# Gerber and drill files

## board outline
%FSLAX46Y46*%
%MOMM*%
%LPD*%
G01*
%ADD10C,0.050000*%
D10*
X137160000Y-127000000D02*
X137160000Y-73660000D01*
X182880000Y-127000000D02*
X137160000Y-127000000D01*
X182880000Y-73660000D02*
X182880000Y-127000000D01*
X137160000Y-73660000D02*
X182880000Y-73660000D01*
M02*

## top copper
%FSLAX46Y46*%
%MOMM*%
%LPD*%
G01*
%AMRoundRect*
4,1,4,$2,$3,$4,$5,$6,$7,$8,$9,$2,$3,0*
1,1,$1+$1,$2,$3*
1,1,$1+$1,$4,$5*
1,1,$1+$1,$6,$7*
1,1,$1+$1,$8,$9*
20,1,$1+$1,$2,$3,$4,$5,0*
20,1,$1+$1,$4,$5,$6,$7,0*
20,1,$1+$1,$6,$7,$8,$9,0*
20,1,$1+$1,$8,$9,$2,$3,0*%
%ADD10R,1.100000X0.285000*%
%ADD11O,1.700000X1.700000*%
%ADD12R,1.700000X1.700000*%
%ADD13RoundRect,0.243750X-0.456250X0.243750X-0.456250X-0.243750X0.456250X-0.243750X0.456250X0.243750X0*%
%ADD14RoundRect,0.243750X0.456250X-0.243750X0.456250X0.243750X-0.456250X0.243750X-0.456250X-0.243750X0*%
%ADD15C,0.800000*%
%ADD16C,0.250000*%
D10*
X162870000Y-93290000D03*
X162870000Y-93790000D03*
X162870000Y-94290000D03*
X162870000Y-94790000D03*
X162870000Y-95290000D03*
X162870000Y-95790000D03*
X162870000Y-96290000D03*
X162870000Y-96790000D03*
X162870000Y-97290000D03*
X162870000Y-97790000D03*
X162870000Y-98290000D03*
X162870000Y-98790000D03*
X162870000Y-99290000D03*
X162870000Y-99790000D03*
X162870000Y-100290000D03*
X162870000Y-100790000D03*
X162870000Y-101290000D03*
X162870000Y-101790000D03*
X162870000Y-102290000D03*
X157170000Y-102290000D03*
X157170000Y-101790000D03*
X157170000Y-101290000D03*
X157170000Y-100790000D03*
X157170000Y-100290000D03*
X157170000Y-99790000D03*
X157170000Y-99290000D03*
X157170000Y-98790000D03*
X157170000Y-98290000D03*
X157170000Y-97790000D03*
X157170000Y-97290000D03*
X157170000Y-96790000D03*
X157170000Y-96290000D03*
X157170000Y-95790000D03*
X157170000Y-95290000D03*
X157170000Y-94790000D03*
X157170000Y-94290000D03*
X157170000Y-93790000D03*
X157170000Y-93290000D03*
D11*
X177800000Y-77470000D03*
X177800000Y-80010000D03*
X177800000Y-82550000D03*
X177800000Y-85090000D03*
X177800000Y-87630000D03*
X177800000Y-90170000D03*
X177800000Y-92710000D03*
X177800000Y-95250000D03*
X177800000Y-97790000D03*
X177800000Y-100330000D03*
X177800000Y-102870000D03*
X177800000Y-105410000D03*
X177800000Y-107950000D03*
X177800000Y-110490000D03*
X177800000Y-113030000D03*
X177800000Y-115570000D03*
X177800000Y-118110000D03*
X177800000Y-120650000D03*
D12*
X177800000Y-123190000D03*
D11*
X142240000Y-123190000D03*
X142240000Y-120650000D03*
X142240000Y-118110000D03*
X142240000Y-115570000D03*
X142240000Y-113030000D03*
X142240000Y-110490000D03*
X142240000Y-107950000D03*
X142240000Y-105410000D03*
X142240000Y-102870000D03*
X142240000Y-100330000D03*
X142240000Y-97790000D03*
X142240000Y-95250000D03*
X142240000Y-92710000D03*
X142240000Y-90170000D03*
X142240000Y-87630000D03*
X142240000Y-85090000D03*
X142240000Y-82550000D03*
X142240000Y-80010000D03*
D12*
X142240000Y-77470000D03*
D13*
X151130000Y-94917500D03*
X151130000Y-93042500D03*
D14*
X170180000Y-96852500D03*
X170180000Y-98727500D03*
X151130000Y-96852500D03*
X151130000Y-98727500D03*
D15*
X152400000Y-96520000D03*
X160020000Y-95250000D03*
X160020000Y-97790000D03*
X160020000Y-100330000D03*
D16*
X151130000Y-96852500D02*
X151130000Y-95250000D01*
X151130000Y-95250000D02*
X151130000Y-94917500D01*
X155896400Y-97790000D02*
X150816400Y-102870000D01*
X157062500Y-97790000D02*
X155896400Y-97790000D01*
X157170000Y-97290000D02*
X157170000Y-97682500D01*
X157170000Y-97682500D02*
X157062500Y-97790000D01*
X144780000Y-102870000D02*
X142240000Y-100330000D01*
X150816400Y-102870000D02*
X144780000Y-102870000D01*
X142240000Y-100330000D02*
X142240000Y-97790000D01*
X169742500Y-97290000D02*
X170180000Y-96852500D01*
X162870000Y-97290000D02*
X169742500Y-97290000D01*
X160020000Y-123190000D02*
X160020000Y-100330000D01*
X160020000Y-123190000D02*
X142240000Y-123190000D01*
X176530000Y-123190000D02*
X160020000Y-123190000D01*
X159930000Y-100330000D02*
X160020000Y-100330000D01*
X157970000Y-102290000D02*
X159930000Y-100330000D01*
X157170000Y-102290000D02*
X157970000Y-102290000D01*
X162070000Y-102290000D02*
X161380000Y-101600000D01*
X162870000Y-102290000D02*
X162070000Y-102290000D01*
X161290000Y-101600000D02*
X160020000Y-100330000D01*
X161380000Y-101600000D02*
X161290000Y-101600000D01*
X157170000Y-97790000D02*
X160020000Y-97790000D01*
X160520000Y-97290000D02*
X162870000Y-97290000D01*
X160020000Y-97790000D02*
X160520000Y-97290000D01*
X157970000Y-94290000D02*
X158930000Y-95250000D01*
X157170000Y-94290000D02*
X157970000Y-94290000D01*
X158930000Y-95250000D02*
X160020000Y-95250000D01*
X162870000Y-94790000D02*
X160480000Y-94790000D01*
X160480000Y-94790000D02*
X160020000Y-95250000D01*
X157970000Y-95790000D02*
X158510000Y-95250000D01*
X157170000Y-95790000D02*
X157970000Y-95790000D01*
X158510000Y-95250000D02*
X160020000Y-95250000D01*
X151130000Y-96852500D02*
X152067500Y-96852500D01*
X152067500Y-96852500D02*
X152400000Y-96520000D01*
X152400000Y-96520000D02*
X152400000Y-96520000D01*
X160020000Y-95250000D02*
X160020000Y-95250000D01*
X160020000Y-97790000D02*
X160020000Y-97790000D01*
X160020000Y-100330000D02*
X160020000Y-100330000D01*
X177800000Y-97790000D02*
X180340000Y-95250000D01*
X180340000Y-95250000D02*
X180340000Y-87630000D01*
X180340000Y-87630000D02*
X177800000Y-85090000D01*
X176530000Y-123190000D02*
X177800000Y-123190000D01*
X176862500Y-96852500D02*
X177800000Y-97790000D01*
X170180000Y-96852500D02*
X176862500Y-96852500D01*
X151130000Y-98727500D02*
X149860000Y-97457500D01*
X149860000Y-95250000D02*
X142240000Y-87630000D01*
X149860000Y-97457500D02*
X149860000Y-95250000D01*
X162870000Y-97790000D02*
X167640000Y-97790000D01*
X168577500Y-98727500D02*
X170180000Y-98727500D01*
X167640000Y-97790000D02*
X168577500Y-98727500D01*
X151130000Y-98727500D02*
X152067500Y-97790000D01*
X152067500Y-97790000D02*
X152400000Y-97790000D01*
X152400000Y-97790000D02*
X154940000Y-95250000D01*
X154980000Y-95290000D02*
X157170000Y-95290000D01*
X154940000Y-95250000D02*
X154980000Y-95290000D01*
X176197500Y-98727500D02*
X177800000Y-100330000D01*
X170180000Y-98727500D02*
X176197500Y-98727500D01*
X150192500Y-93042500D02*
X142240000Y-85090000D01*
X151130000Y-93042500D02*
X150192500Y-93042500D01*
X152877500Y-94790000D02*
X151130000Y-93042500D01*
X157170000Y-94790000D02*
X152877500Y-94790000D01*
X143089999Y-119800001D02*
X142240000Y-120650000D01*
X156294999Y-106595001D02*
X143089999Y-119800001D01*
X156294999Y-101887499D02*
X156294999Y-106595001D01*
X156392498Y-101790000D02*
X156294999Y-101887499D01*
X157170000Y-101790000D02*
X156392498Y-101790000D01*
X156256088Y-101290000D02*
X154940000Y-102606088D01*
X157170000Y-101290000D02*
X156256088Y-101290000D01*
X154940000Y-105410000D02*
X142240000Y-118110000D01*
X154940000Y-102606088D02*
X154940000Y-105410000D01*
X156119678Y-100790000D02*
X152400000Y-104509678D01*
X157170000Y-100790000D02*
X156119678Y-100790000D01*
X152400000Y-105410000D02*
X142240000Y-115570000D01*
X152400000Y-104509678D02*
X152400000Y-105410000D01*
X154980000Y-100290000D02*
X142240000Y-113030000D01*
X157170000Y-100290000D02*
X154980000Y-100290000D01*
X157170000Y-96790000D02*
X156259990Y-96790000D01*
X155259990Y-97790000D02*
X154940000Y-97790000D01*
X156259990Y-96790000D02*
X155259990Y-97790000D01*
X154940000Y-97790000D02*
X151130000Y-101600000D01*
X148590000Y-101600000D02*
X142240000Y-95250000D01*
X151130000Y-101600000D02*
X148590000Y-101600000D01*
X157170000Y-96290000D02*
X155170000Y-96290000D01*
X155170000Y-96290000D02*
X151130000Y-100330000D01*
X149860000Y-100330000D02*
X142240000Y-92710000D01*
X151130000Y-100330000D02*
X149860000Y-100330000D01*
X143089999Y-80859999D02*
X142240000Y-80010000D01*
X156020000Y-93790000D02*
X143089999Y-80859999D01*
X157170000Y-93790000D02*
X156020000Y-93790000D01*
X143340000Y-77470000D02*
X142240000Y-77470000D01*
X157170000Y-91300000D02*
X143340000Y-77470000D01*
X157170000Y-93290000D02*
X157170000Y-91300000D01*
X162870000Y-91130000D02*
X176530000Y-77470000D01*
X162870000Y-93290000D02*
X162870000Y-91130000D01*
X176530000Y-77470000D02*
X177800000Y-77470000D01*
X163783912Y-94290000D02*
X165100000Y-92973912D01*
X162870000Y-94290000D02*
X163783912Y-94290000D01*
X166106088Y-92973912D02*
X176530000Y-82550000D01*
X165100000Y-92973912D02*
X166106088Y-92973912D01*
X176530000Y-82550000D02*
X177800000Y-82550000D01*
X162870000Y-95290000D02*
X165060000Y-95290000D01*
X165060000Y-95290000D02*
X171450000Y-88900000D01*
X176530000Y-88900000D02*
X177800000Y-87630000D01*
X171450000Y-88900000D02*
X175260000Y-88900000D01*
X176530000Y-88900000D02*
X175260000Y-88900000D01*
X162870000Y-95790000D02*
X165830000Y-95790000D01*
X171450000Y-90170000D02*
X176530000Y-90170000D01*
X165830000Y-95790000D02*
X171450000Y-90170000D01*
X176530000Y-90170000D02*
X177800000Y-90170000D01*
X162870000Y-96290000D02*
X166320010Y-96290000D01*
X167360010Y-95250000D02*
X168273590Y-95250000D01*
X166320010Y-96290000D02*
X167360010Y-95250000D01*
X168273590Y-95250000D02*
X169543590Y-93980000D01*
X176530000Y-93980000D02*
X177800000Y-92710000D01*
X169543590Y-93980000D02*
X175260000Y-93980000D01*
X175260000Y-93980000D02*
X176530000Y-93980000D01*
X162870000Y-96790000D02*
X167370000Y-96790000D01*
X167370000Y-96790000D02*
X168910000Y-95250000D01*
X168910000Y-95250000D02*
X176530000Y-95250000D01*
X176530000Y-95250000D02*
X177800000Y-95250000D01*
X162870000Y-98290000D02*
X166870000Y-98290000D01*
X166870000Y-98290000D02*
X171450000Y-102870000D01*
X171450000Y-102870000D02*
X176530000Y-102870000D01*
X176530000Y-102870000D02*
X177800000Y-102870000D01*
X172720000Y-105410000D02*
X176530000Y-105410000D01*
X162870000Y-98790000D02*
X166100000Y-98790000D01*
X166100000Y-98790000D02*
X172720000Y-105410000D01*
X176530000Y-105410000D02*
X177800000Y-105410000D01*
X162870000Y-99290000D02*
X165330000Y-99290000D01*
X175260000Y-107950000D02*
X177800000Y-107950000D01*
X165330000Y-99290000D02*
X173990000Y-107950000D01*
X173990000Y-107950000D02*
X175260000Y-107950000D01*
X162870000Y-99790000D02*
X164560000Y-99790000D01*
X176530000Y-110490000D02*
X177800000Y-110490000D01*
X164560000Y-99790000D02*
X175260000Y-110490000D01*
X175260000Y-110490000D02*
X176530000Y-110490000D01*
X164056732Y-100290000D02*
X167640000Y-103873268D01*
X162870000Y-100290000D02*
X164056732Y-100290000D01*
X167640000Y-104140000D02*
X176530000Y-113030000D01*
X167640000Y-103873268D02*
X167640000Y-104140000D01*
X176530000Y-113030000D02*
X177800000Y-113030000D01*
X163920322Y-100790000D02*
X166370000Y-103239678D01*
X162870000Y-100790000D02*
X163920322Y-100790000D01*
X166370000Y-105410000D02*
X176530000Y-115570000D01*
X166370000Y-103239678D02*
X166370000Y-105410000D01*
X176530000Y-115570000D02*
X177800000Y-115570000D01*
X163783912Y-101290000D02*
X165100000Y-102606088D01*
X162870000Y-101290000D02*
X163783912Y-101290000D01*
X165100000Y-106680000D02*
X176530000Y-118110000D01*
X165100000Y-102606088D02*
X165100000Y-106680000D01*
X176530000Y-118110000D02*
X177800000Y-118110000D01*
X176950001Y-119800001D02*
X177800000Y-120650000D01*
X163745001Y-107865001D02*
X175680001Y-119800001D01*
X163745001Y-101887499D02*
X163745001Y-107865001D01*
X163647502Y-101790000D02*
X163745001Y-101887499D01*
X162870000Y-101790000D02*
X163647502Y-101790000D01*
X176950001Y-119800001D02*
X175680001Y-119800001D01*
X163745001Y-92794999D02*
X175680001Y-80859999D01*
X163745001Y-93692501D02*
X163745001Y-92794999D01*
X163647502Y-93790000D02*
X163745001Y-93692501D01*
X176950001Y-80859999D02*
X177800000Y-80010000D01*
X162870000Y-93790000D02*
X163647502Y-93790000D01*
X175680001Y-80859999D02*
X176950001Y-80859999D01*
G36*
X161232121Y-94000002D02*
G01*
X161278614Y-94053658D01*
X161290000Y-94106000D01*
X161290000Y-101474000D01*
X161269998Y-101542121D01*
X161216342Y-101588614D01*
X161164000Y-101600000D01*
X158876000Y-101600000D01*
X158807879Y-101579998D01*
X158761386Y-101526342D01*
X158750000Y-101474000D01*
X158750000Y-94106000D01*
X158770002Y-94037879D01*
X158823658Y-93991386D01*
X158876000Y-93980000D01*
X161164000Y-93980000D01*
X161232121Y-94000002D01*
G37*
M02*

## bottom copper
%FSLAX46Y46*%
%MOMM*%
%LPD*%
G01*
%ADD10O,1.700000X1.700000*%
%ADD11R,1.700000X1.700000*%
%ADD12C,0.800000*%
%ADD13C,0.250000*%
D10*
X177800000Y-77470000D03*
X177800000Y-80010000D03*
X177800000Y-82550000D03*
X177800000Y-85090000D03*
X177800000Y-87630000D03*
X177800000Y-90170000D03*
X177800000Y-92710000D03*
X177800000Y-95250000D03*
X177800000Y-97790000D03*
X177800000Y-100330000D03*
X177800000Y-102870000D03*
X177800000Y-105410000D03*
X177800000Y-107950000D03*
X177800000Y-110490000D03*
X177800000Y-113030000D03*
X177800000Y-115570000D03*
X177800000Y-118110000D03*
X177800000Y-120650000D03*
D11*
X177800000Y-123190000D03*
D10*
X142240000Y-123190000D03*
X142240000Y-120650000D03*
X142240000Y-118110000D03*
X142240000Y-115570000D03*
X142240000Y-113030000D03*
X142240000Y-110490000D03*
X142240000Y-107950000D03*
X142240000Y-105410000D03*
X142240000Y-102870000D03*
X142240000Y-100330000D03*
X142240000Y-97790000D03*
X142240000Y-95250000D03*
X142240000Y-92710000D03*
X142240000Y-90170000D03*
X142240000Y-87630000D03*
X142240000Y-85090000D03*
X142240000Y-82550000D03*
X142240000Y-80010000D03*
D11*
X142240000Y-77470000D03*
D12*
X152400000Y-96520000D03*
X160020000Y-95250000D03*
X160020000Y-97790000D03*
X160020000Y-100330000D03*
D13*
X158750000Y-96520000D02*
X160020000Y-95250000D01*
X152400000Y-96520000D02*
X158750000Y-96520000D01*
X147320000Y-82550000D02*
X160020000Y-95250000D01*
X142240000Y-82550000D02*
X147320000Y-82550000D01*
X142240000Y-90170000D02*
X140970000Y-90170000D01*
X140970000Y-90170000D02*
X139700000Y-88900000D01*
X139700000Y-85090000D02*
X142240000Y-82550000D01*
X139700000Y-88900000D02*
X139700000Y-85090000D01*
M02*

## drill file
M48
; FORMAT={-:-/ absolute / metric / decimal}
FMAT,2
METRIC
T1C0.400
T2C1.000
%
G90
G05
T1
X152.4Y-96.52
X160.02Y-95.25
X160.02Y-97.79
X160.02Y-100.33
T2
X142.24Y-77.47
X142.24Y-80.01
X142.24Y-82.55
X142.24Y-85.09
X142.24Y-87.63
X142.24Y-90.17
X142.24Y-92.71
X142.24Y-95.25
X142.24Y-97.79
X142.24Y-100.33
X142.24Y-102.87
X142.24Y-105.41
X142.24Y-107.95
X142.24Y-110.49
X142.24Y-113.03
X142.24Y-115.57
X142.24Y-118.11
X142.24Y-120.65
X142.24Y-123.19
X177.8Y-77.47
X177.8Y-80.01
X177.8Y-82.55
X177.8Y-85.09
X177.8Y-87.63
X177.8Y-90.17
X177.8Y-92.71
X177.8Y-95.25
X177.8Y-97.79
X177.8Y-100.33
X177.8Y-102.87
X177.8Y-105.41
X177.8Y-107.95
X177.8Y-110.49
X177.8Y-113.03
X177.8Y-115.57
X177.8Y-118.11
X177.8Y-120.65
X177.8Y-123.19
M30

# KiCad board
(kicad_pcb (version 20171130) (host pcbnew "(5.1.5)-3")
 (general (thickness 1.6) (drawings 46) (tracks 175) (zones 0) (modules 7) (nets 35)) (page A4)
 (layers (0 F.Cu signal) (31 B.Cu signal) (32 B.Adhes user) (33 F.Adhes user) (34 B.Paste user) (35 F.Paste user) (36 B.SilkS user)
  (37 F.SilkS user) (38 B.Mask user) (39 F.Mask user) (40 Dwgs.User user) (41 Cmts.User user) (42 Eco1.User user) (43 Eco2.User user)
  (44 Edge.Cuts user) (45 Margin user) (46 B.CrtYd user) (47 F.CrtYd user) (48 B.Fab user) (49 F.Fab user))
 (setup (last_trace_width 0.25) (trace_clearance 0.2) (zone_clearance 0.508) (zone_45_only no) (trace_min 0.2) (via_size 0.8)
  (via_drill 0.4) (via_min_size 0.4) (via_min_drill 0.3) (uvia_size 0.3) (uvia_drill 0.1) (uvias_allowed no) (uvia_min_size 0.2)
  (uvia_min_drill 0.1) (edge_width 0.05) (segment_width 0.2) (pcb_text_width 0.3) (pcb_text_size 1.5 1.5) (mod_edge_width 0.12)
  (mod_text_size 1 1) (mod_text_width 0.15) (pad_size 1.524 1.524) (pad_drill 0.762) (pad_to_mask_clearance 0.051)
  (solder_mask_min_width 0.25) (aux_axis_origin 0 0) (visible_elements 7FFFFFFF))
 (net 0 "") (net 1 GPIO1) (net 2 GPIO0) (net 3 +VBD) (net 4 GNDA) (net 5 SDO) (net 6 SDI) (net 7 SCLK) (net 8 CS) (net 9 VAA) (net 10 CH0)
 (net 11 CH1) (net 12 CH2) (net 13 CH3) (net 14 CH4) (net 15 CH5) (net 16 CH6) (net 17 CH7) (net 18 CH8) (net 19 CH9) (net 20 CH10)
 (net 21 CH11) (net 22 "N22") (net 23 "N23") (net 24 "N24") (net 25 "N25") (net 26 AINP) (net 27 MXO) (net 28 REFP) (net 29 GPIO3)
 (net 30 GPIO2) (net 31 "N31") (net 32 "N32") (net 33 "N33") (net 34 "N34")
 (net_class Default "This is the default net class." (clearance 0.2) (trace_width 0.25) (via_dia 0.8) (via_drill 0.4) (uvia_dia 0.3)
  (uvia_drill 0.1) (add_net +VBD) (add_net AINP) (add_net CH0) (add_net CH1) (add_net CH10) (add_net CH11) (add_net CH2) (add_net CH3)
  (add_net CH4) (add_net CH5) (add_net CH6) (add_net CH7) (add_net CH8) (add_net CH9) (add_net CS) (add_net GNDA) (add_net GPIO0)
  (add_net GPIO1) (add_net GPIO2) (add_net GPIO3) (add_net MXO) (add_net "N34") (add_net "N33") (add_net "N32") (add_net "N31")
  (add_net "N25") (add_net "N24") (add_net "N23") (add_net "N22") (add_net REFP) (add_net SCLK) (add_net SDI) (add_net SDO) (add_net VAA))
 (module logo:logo (layer F.Cu) (at 160.02 82.55)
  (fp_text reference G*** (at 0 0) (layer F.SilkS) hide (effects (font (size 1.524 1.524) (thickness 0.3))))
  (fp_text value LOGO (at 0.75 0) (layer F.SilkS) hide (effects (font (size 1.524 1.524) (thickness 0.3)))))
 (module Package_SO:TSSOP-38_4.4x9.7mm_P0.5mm (layer F.Cu) (at 160.02 97.79)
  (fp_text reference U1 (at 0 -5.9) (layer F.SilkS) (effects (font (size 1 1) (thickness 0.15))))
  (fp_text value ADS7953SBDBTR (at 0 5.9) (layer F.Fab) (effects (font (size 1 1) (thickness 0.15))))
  (pad 38 smd rect (at 2.85 -4.5) (size 1.1 0.285) (layers F.Cu F.Paste F.Mask) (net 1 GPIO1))
  (pad 37 smd rect (at 2.85 -4) (size 1.1 0.285) (layers F.Cu F.Paste F.Mask) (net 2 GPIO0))
  (pad 36 smd rect (at 2.85 -3.5) (size 1.1 0.285) (layers F.Cu F.Paste F.Mask) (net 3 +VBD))
  (pad 35 smd rect (at 2.85 -3) (size 1.1 0.285) (layers F.Cu F.Paste F.Mask) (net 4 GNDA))
  (pad 34 smd rect (at 2.85 -2.5) (size 1.1 0.285) (layers F.Cu F.Paste F.Mask) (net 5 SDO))
  (pad 33 smd rect (at 2.85 -2) (size 1.1 0.285) (layers F.Cu F.Paste F.Mask) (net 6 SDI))
  (pad 32 smd rect (at 2.85 -1.5) (size 1.1 0.285) (layers F.Cu F.Paste F.Mask) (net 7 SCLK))
  (pad 31 smd rect (at 2.85 -1) (size 1.1 0.285) (layers F.Cu F.Paste F.Mask) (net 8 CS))
  (pad 30 smd rect (at 2.85 -0.5) (size 1.1 0.285) (layers F.Cu F.Paste F.Mask) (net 4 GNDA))
  (pad 29 smd rect (at 2.85 0) (size 1.1 0.285) (layers F.Cu F.Paste F.Mask) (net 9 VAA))
  (pad 28 smd rect (at 2.85 0.5) (size 1.1 0.285) (layers F.Cu F.Paste F.Mask) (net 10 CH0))
  (pad 27 smd rect (at 2.85 1) (size 1.1 0.285) (layers F.Cu F.Paste F.Mask) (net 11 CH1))
  (pad 26 smd rect (at 2.85 1.5) (size 1.1 0.285) (layers F.Cu F.Paste F.Mask) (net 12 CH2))
  (pad 25 smd rect (at 2.85 2) (size 1.1 0.285) (layers F.Cu F.Paste F.Mask) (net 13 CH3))
  (pad 24 smd rect (at 2.85 2.5) (size 1.1 0.285) (layers F.Cu F.Paste F.Mask) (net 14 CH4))
  (pad 23 smd rect (at 2.85 3) (size 1.1 0.285) (layers F.Cu F.Paste F.Mask) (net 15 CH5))
  (pad 22 smd rect (at 2.85 3.5) (size 1.1 0.285) (layers F.Cu F.Paste F.Mask) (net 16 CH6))
  (pad 21 smd rect (at 2.85 4) (size 1.1 0.285) (layers F.Cu F.Paste F.Mask) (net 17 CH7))
  (pad 20 smd rect (at 2.85 4.5) (size 1.1 0.285) (layers F.Cu F.Paste F.Mask) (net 4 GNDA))
  (pad 19 smd rect (at -2.85 4.5) (size 1.1 0.285) (layers F.Cu F.Paste F.Mask) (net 4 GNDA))
  (pad 18 smd rect (at -2.85 4) (size 1.1 0.285) (layers F.Cu F.Paste F.Mask) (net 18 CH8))
  (pad 17 smd rect (at -2.85 3.5) (size 1.1 0.285) (layers F.Cu F.Paste F.Mask) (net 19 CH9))
  (pad 16 smd rect (at -2.85 3) (size 1.1 0.285) (layers F.Cu F.Paste F.Mask) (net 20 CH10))
  (pad 15 smd rect (at -2.85 2.5) (size 1.1 0.285) (layers F.Cu F.Paste F.Mask) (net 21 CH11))
  (pad 14 smd rect (at -2.85 2) (size 1.1 0.285) (layers F.Cu F.Paste F.Mask) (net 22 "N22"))
  (pad 13 smd rect (at -2.85 1.5) (size 1.1 0.285) (layers F.Cu F.Paste F.Mask) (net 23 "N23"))
  (pad 12 smd rect (at -2.85 1) (size 1.1 0.285) (layers F.Cu F.Paste F.Mask) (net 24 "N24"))
  (pad 11 smd rect (at -2.85 0.5) (size 1.1 0.285) (layers F.Cu F.Paste F.Mask) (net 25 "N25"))
  (pad 10 smd rect (at -2.85 0) (size 1.1 0.285) (layers F.Cu F.Paste F.Mask) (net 4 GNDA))
  (pad 9 smd rect (at -2.85 -0.5) (size 1.1 0.285) (layers F.Cu F.Paste F.Mask) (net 4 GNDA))
  (pad 8 smd rect (at -2.85 -1) (size 1.1 0.285) (layers F.Cu F.Paste F.Mask) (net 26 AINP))
  (pad 7 smd rect (at -2.85 -1.5) (size 1.1 0.285) (layers F.Cu F.Paste F.Mask) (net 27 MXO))
  (pad 6 smd rect (at -2.85 -2) (size 1.1 0.285) (layers F.Cu F.Paste F.Mask) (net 4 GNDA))
  (pad 5 smd rect (at -2.85 -2.5) (size 1.1 0.285) (layers F.Cu F.Paste F.Mask) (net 9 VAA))
  (pad 4 smd rect (at -2.85 -3) (size 1.1 0.285) (layers F.Cu F.Paste F.Mask) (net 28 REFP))
  (pad 3 smd rect (at -2.85 -3.5) (size 1.1 0.285) (layers F.Cu F.Paste F.Mask) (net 4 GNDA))
  (pad 2 smd rect (at -2.85 -4) (size 1.1 0.285) (layers F.Cu F.Paste F.Mask) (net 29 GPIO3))
  (pad 1 smd rect (at -2.85 -4.5) (size 1.1 0.285) (layers F.Cu F.Paste F.Mask) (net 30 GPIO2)))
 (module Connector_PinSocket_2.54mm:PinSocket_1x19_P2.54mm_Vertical (layer F.Cu) (at 177.8 123.19 180)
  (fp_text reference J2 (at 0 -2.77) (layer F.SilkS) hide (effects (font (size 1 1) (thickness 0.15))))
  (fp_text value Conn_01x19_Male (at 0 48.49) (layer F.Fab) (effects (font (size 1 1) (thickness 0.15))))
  (pad 19 thru_hole oval (at 0 45.72 180) (size 1.7 1.7) (drill 1) (layers *.Cu *.Mask) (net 1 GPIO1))
  (pad 18 thru_hole oval (at 0 43.18 180) (size 1.7 1.7) (drill 1) (layers *.Cu *.Mask) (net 2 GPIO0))
  (pad 17 thru_hole oval (at 0 40.64 180) (size 1.7 1.7) (drill 1) (layers *.Cu *.Mask) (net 3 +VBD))
  (pad 16 thru_hole oval (at 0 38.1 180) (size 1.7 1.7) (drill 1) (layers *.Cu *.Mask) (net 4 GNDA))
  (pad 15 thru_hole oval (at 0 35.56 180) (size 1.7 1.7) (drill 1) (layers *.Cu *.Mask) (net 5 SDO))
  (pad 14 thru_hole oval (at 0 33.02 180) (size 1.7 1.7) (drill 1) (layers *.Cu *.Mask) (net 6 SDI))
  (pad 13 thru_hole oval (at 0 30.48 180) (size 1.7 1.7) (drill 1) (layers *.Cu *.Mask) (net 7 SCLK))
  (pad 12 thru_hole oval (at 0 27.94 180) (size 1.7 1.7) (drill 1) (layers *.Cu *.Mask) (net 8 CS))
  (pad 11 thru_hole oval (at 0 25.4 180) (size 1.7 1.7) (drill 1) (layers *.Cu *.Mask) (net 4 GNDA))
  (pad 10 thru_hole oval (at 0 22.86 180) (size 1.7 1.7) (drill 1) (layers *.Cu *.Mask) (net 9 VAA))
  (pad 9 thru_hole oval (at 0 20.32 180) (size 1.7 1.7) (drill 1) (layers *.Cu *.Mask) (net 10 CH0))
  (pad 8 thru_hole oval (at 0 17.78 180) (size 1.7 1.7) (drill 1) (layers *.Cu *.Mask) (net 11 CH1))
  (pad 7 thru_hole oval (at 0 15.24 180) (size 1.7 1.7) (drill 1) (layers *.Cu *.Mask) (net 12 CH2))
  (pad 6 thru_hole oval (at 0 12.7 180) (size 1.7 1.7) (drill 1) (layers *.Cu *.Mask) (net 13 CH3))
  (pad 5 thru_hole oval (at 0 10.16 180) (size 1.7 1.7) (drill 1) (layers *.Cu *.Mask) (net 14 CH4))
  (pad 4 thru_hole oval (at 0 7.62 180) (size 1.7 1.7) (drill 1) (layers *.Cu *.Mask) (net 15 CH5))
  (pad 3 thru_hole oval (at 0 5.08 180) (size 1.7 1.7) (drill 1) (layers *.Cu *.Mask) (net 16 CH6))
  (pad 2 thru_hole oval (at 0 2.54 180) (size 1.7 1.7) (drill 1) (layers *.Cu *.Mask) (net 17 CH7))
  (pad 1 thru_hole rect (at 0 0 180) (size 1.7 1.7) (drill 1) (layers *.Cu *.Mask) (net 4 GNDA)))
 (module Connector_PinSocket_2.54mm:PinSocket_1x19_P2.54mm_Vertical (layer F.Cu) (at 142.24 77.47)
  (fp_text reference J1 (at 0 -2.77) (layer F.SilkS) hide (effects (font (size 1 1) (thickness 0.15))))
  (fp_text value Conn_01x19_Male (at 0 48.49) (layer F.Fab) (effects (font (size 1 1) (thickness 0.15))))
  (pad 19 thru_hole oval (at 0 45.72) (size 1.7 1.7) (drill 1) (layers *.Cu *.Mask) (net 4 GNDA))
  (pad 18 thru_hole oval (at 0 43.18) (size 1.7 1.7) (drill 1) (layers *.Cu *.Mask) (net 18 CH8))
  (pad 17 thru_hole oval (at 0 40.64) (size 1.7 1.7) (drill 1) (layers *.Cu *.Mask) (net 19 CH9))
  (pad 16 thru_hole oval (at 0 38.1) (size 1.7 1.7) (drill 1) (layers *.Cu *.Mask) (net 20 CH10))
  (pad 15 thru_hole oval (at 0 35.56) (size 1.7 1.7) (drill 1) (layers *.Cu *.Mask) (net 21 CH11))
  (pad 14 thru_hole oval (at 0 33.02) (size 1.7 1.7) (drill 1) (layers *.Cu *.Mask) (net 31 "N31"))
  (pad 13 thru_hole oval (at 0 30.48) (size 1.7 1.7) (drill 1) (layers *.Cu *.Mask) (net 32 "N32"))
  (pad 12 thru_hole oval (at 0 27.94) (size 1.7 1.7) (drill 1) (layers *.Cu *.Mask) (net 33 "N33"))
  (pad 11 thru_hole oval (at 0 25.4) (size 1.7 1.7) (drill 1) (layers *.Cu *.Mask) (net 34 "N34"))
  (pad 10 thru_hole oval (at 0 22.86) (size 1.7 1.7) (drill 1) (layers *.Cu *.Mask) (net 4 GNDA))
  (pad 9 thru_hole oval (at 0 20.32) (size 1.7 1.7) (drill 1) (layers *.Cu *.Mask) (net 4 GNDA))
  (pad 8 thru_hole oval (at 0 17.78) (size 1.7 1.7) (drill 1) (layers *.Cu *.Mask) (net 26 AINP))
  (pad 7 thru_hole oval (at 0 15.24) (size 1.7 1.7) (drill 1) (layers *.Cu *.Mask) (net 27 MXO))
  (pad 6 thru_hole oval (at 0 12.7) (size 1.7 1.7) (drill 1) (layers *.Cu *.Mask) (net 4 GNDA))
  (pad 5 thru_hole oval (at 0 10.16) (size 1.7 1.7) (drill 1) (layers *.Cu *.Mask) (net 9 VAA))
  (pad 4 thru_hole oval (at 0 7.62) (size 1.7 1.7) (drill 1) (layers *.Cu *.Mask) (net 28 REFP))
  (pad 3 thru_hole oval (at 0 5.08) (size 1.7 1.7) (drill 1) (layers *.Cu *.Mask) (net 4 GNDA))
  (pad 2 thru_hole oval (at 0 2.54) (size 1.7 1.7) (drill 1) (layers *.Cu *.Mask) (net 29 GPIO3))
  (pad 1 thru_hole rect (at 0 0) (size 1.7 1.7) (drill 1) (layers *.Cu *.Mask) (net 30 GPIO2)))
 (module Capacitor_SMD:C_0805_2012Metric (layer F.Cu) (at 151.13 93.98 270)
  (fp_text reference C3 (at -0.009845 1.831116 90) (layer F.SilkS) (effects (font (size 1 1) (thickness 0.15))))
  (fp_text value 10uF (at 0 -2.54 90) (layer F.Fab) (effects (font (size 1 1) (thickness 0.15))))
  (pad 2 smd roundrect (at 0.9375 0 270) (size 0.975 1.4) (layers F.Cu F.Paste F.Mask) (roundrect_rratio 0.25) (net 4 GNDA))
  (pad 1 smd roundrect (at -0.9375 0 270) (size 0.975 1.4) (layers F.Cu F.Paste F.Mask) (roundrect_rratio 0.25) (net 28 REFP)))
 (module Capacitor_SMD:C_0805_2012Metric (layer F.Cu) (at 170.18 97.79 90)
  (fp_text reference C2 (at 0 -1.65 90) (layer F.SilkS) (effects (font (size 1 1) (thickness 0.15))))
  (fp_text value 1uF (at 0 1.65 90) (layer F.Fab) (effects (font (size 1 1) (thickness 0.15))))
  (pad 2 smd roundrect (at 0.9375 0 90) (size 0.975 1.4) (layers F.Cu F.Paste F.Mask) (roundrect_rratio 0.25) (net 4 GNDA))
  (pad 1 smd roundrect (at -0.9375 0 90) (size 0.975 1.4) (layers F.Cu F.Paste F.Mask) (roundrect_rratio 0.25) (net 9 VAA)))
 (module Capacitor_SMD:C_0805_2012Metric (layer F.Cu) (at 151.13 97.79 90)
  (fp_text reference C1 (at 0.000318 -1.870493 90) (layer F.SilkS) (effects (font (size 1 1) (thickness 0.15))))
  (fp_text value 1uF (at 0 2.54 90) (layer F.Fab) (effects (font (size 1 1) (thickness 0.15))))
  (pad 2 smd roundrect (at 0.9375 0 90) (size 0.975 1.4) (layers F.Cu F.Paste F.Mask) (roundrect_rratio 0.25) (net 4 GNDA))
  (pad 1 smd roundrect (at -0.9375 0 90) (size 0.975 1.4) (layers F.Cu F.Paste F.Mask) (roundrect_rratio 0.25) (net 9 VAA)))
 (gr_line (start 137.16 127) (end 137.16 73.66) (layer Edge.Cuts) (width 0.05))
 (gr_line (start 182.88 127) (end 137.16 127) (layer Edge.Cuts) (width 0.05))
 (gr_line (start 182.88 73.66) (end 182.88 127) (layer Edge.Cuts) (width 0.05))
 (gr_line (start 137.16 73.66) (end 182.88 73.66) (layer Edge.Cuts) (width 0.05))
 (segment (start 151.13 96.8525) (end 151.13 95.25) (width 0.25) (layer F.Cu) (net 4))
 (segment (start 151.13 95.25) (end 151.13 94.9175) (width 0.25) (layer F.Cu) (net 4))
 (segment (start 155.8964 97.79) (end 150.8164 102.87) (width 0.25) (layer F.Cu) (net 4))
 (segment (start 157.0625 97.79) (end 155.8964 97.79) (width 0.25) (layer F.Cu) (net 4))
 (segment (start 157.17 97.29) (end 157.17 97.6825) (width 0.25) (layer F.Cu) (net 4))
 (segment (start 157.17 97.6825) (end 157.0625 97.79) (width 0.25) (layer F.Cu) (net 4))
 (segment (start 144.78 102.87) (end 142.24 100.33) (width 0.25) (layer F.Cu) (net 4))
 (segment (start 150.8164 102.87) (end 144.78 102.87) (width 0.25) (layer F.Cu) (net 4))
 (segment (start 142.24 100.33) (end 142.24 97.79) (width 0.25) (layer F.Cu) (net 4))
 (segment (start 169.7425 97.29) (end 170.18 96.8525) (width 0.25) (layer F.Cu) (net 4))
 (segment (start 162.87 97.29) (end 169.7425 97.29) (width 0.25) (layer F.Cu) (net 4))
 (segment (start 160.02 123.19) (end 160.02 100.33) (width 0.25) (layer F.Cu) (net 4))
 (segment (start 160.02 123.19) (end 142.24 123.19) (width 0.25) (layer F.Cu) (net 4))
 (segment (start 176.53 123.19) (end 160.02 123.19) (width 0.25) (layer F.Cu) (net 4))
 (segment (start 159.93 100.33) (end 160.02 100.33) (width 0.25) (layer F.Cu) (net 4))
 (segment (start 157.97 102.29) (end 159.93 100.33) (width 0.25) (layer F.Cu) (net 4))
 (segment (start 157.17 102.29) (end 157.97 102.29) (width 0.25) (layer F.Cu) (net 4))
 (segment (start 162.07 102.29) (end 161.38 101.6) (width 0.25) (layer F.Cu) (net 4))
 (segment (start 162.87 102.29) (end 162.07 102.29) (width 0.25) (layer F.Cu) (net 4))
 (segment (start 161.29 101.6) (end 160.02 100.33) (width 0.25) (layer F.Cu) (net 4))
 (segment (start 161.38 101.6) (end 161.29 101.6) (width 0.25) (layer F.Cu) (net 4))
 (segment (start 157.17 97.79) (end 160.02 97.79) (width 0.25) (layer F.Cu) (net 4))
 (segment (start 160.52 97.29) (end 162.87 97.29) (width 0.25) (layer F.Cu) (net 4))
 (segment (start 160.02 97.79) (end 160.52 97.29) (width 0.25) (layer F.Cu) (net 4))
 (segment (start 157.97 94.29) (end 158.93 95.25) (width 0.25) (layer F.Cu) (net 4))
 (segment (start 157.17 94.29) (end 157.97 94.29) (width 0.25) (layer F.Cu) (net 4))
 (segment (start 158.93 95.25) (end 160.02 95.25) (width 0.25) (layer F.Cu) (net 4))
 (segment (start 162.87 94.79) (end 160.48 94.79) (width 0.25) (layer F.Cu) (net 4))
 (segment (start 160.48 94.79) (end 160.02 95.25) (width 0.25) (layer F.Cu) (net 4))
 (segment (start 157.97 95.79) (end 158.51 95.25) (width 0.25) (layer F.Cu) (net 4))
 (segment (start 157.17 95.79) (end 157.97 95.79) (width 0.25) (layer F.Cu) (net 4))
 (segment (start 158.51 95.25) (end 160.02 95.25) (width 0.25) (layer F.Cu) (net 4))
 (segment (start 151.13 96.8525) (end 152.0675 96.8525) (width 0.25) (layer F.Cu) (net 4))
 (segment (start 152.0675 96.8525) (end 152.4 96.52) (width 0.25) (layer F.Cu) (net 4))
 (segment (start 152.4 96.52) (end 152.4 96.52) (width 0.25) (layer F.Cu) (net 4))
 (via (at 152.4 96.52) (size 0.8) (drill 0.4) (layers F.Cu B.Cu) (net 4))
 (segment (start 160.02 95.25) (end 160.02 95.25) (width 0.25) (layer F.Cu) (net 4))
 (via (at 160.02 95.25) (size 0.8) (drill 0.4) (layers F.Cu B.Cu) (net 4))
 (segment (start 160.02 97.79) (end 160.02 97.79) (width 0.25) (layer F.Cu) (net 4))
 (via (at 160.02 97.79) (size 0.8) (drill 0.4) (layers F.Cu B.Cu) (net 4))
 (segment (start 160.02 100.33) (end 160.02 100.33) (width 0.25) (layer F.Cu) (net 4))
 (via (at 160.02 100.33) (size 0.8) (drill 0.4) (layers F.Cu B.Cu) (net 4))
 (segment (start 158.75 96.52) (end 160.02 95.25) (width 0.25) (layer B.Cu) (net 4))
 (segment (start 152.4 96.52) (end 158.75 96.52) (width 0.25) (layer B.Cu) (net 4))
 (segment (start 147.32 82.55) (end 160.02 95.25) (width 0.25) (layer B.Cu) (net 4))
 (segment (start 142.24 82.55) (end 147.32 82.55) (width 0.25) (layer B.Cu) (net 4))
 (segment (start 142.24 90.17) (end 140.97 90.17) (width 0.25) (layer B.Cu) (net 4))
 (segment (start 140.97 90.17) (end 139.7 88.9) (width 0.25) (layer B.Cu) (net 4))
 (segment (start 139.7 85.09) (end 142.24 82.55) (width 0.25) (layer B.Cu) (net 4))
 (segment (start 139.7 88.9) (end 139.7 85.09) (width 0.25) (layer B.Cu) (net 4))
 (segment (start 177.8 97.79) (end 180.34 95.25) (width 0.25) (layer F.Cu) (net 4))
 (segment (start 180.34 95.25) (end 180.34 87.63) (width 0.25) (layer F.Cu) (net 4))
 (segment (start 180.34 87.63) (end 177.8 85.09) (width 0.25) (layer F.Cu) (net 4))
 (segment (start 176.53 123.19) (end 177.8 123.19) (width 0.25) (layer F.Cu) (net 4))
 (segment (start 176.8625 96.8525) (end 177.8 97.79) (width 0.25) (layer F.Cu) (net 4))
 (segment (start 170.18 96.8525) (end 176.8625 96.8525) (width 0.25) (layer F.Cu) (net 4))
 (segment (start 151.13 98.7275) (end 149.86 97.4575) (width 0.25) (layer F.Cu) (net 9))
 (segment (start 149.86 95.25) (end 142.24 87.63) (width 0.25) (layer F.Cu) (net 9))
 (segment (start 149.86 97.4575) (end 149.86 95.25) (width 0.25) (layer F.Cu) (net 9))
 (segment (start 162.87 97.79) (end 167.64 97.79) (width 0.25) (layer F.Cu) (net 9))
 (segment (start 168.5775 98.7275) (end 170.18 98.7275) (width 0.25) (layer F.Cu) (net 9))
 (segment (start 167.64 97.79) (end 168.5775 98.7275) (width 0.25) (layer F.Cu) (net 9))
 (segment (start 151.13 98.7275) (end 152.0675 97.79) (width 0.25) (layer F.Cu) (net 9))
 (segment (start 152.0675 97.79) (end 152.4 97.79) (width 0.25) (layer F.Cu) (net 9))
 (segment (start 152.4 97.79) (end 154.94 95.25) (width 0.25) (layer F.Cu) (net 9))
 (segment (start 154.98 95.29) (end 157.17 95.29) (width 0.25) (layer F.Cu) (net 9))
 (segment (start 154.94 95.25) (end 154.98 95.29) (width 0.25) (layer F.Cu) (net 9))
 (segment (start 176.1975 98.7275) (end 177.8 100.33) (width 0.25) (layer F.Cu) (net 9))
 (segment (start 170.18 98.7275) (end 176.1975 98.7275) (width 0.25) (layer F.Cu) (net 9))
 (segment (start 150.1925 93.0425) (end 142.24 85.09) (width 0.25) (layer F.Cu) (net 28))
 (segment (start 151.13 93.0425) (end 150.1925 93.0425) (width 0.25) (layer F.Cu) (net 28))
 (segment (start 152.8775 94.79) (end 151.13 93.0425) (width 0.25) (layer F.Cu) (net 28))
 (segment (start 157.17 94.79) (end 152.8775 94.79) (width 0.25) (layer F.Cu) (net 28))
 (segment (start 143.089999 119.800001) (end 142.24 120.65) (width 0.25) (layer F.Cu) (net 18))
 (segment (start 156.294999 106.595001) (end 143.089999 119.800001) (width 0.25) (layer F.Cu) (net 18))
 (segment (start 156.294999 101.887499) (end 156.294999 106.595001) (width 0.25) (layer F.Cu) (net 18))
 (segment (start 156.392498 101.79) (end 156.294999 101.887499) (width 0.25) (layer F.Cu) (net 18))
 (segment (start 157.17 101.79) (end 156.392498 101.79) (width 0.25) (layer F.Cu) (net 18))
 (segment (start 156.256088 101.29) (end 154.94 102.606088) (width 0.25) (layer F.Cu) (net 19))
 (segment (start 157.17 101.29) (end 156.256088 101.29) (width 0.25) (layer F.Cu) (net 19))
 (segment (start 154.94 105.41) (end 142.24 118.11) (width 0.25) (layer F.Cu) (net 19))
 (segment (start 154.94 102.606088) (end 154.94 105.41) (width 0.25) (layer F.Cu) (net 19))
 (segment (start 156.119678 100.79) (end 152.4 104.509678) (width 0.25) (layer F.Cu) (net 20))
 (segment (start 157.17 100.79) (end 156.119678 100.79) (width 0.25) (layer F.Cu) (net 20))
 (segment (start 152.4 105.41) (end 142.24 115.57) (width 0.25) (layer F.Cu) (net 20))
 (segment (start 152.4 104.509678) (end 152.4 105.41) (width 0.25) (layer F.Cu) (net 20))
 (segment (start 154.98 100.29) (end 142.24 113.03) (width 0.25) (layer F.Cu) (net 21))
 (segment (start 157.17 100.29) (end 154.98 100.29) (width 0.25) (layer F.Cu) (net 21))
 (segment (start 157.17 96.79) (end 156.25999 96.79) (width 0.25) (layer F.Cu) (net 26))
 (segment (start 155.25999 97.79) (end 154.94 97.79) (width 0.25) (layer F.Cu) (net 26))
 (segment (start 156.25999 96.79) (end 155.25999 97.79) (width 0.25) (layer F.Cu) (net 26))
 (segment (start 154.94 97.79) (end 151.13 101.6) (width 0.25) (layer F.Cu) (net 26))
 (segment (start 148.59 101.6) (end 142.24 95.25) (width 0.25) (layer F.Cu) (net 26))
 (segment (start 151.13 101.6) (end 148.59 101.6) (width 0.25) (layer F.Cu) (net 26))
 (segment (start 157.17 96.29) (end 155.17 96.29) (width 0.25) (layer F.Cu) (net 27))
 (segment (start 155.17 96.29) (end 151.13 100.33) (width 0.25) (layer F.Cu) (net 27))
 (segment (start 149.86 100.33) (end 142.24 92.71) (width 0.25) (layer F.Cu) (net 27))
 (segment (start 151.13 100.33) (end 149.86 100.33) (width 0.25) (layer F.Cu) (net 27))
 (segment (start 143.089999 80.859999) (end 142.24 80.01) (width 0.25) (layer F.Cu) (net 29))
 (segment (start 156.02 93.79) (end 143.089999 80.859999) (width 0.25) (layer F.Cu) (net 29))
 (segment (start 157.17 93.79) (end 156.02 93.79) (width 0.25) (layer F.Cu) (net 29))
 (segment (start 143.34 77.47) (end 142.24 77.47) (width 0.25) (layer F.Cu) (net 30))
 (segment (start 157.17 91.3) (end 143.34 77.47) (width 0.25) (layer F.Cu) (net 30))
 (segment (start 157.17 93.29) (end 157.17 91.3) (width 0.25) (layer F.Cu) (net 30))
 (segment (start 162.87 91.13) (end 176.53 77.47) (width 0.25) (layer F.Cu) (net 1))
 (segment (start 162.87 93.29) (end 162.87 91.13) (width 0.25) (layer F.Cu) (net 1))
 (segment (start 176.53 77.47) (end 177.8 77.47) (width 0.25) (layer F.Cu) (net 1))
 (segment (start 163.783912 94.29) (end 165.1 92.973912) (width 0.25) (layer F.Cu) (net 3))
 (segment (start 162.87 94.29) (end 163.783912 94.29) (width 0.25) (layer F.Cu) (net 3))
 (segment (start 166.106088 92.973912) (end 176.53 82.55) (width 0.25) (layer F.Cu) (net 3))
 (segment (start 165.1 92.973912) (end 166.106088 92.973912) (width 0.25) (layer F.Cu) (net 3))
 (segment (start 176.53 82.55) (end 177.8 82.55) (width 0.25) (layer F.Cu) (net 3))
 (segment (start 162.87 95.29) (end 165.06 95.29) (width 0.25) (layer F.Cu) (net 5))
 (segment (start 165.06 95.29) (end 171.45 88.9) (width 0.25) (layer F.Cu) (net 5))
 (segment (start 176.53 88.9) (end 177.8 87.63) (width 0.25) (layer F.Cu) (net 5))
 (segment (start 171.45 88.9) (end 175.26 88.9) (width 0.25) (layer F.Cu) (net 5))
 (segment (start 176.53 88.9) (end 175.26 88.9) (width 0.25) (layer F.Cu) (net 5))
 (segment (start 162.87 95.79) (end 165.83 95.79) (width 0.25) (layer F.Cu) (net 6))
 (segment (start 171.45 90.17) (end 176.53 90.17) (width 0.25) (layer F.Cu) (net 6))
 (segment (start 165.83 95.79) (end 171.45 90.17) (width 0.25) (layer F.Cu) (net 6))
 (segment (start 176.53 90.17) (end 177.8 90.17) (width 0.25) (layer F.Cu) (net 6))
 (segment (start 162.87 96.29) (end 166.32001 96.29) (width 0.25) (layer F.Cu) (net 7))
 (segment (start 167.36001 95.25) (end 168.27359 95.25) (width 0.25) (layer F.Cu) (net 7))
 (segment (start 166.32001 96.29) (end 167.36001 95.25) (width 0.25) (layer F.Cu) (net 7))
 (segment (start 168.27359 95.25) (end 169.54359 93.98) (width 0.25) (layer F.Cu) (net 7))
 (segment (start 176.53 93.98) (end 177.8 92.71) (width 0.25) (layer F.Cu) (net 7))
 (segment (start 169.54359 93.98) (end 175.26 93.98) (width 0.25) (layer F.Cu) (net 7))
 (segment (start 175.26 93.98) (end 176.53 93.98) (width 0.25) (layer F.Cu) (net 7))
 (segment (start 162.87 96.79) (end 167.37 96.79) (width 0.25) (layer F.Cu) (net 8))
 (segment (start 167.37 96.79) (end 168.91 95.25) (width 0.25) (layer F.Cu) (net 8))
 (segment (start 168.91 95.25) (end 176.53 95.25) (width 0.25) (layer F.Cu) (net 8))
 (segment (start 176.53 95.25) (end 177.8 95.25) (width 0.25) (layer F.Cu) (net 8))
 (segment (start 162.87 98.29) (end 166.87 98.29) (width 0.25) (layer F.Cu) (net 10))
 (segment (start 166.87 98.29) (end 171.45 102.87) (width 0.25) (layer F.Cu) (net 10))
 (segment (start 171.45 102.87) (end 176.53 102.87) (width 0.25) (layer F.Cu) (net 10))
 (segment (start 176.53 102.87) (end 177.8 102.87) (width 0.25) (layer F.Cu) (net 10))
 (segment (start 172.72 105.41) (end 176.53 105.41) (width 0.25) (layer F.Cu) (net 11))
 (segment (start 162.87 98.79) (end 166.1 98.79) (width 0.25) (layer F.Cu) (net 11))
 (segment (start 166.1 98.79) (end 172.72 105.41) (width 0.25) (layer F.Cu) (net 11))
 (segment (start 176.53 105.41) (end 177.8 105.41) (width 0.25) (layer F.Cu) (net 11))
 (segment (start 162.87 99.29) (end 165.33 99.29) (width 0.25) (layer F.Cu) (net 12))
 (segment (start 175.26 107.95) (end 177.8 107.95) (width 0.25) (layer F.Cu) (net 12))
 (segment (start 165.33 99.29) (end 173.99 107.95) (width 0.25) (layer F.Cu) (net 12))
 (segment (start 173.99 107.95) (end 175.26 107.95) (width 0.25) (layer F.Cu) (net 12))
 (segment (start 162.87 99.79) (end 164.56 99.79) (width 0.25) (layer F.Cu) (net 13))
 (segment (start 176.53 110.49) (end 177.8 110.49) (width 0.25) (layer F.Cu) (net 13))
 (segment (start 164.56 99.79) (end 175.26 110.49) (width 0.25) (layer F.Cu) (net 13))
 (segment (start 175.26 110.49) (end 176.53 110.49) (width 0.25) (layer F.Cu) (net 13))
 (segment (start 164.056732 100.29) (end 167.64 103.873268) (width 0.25) (layer F.Cu) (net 14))
 (segment (start 162.87 100.29) (end 164.056732 100.29) (width 0.25) (layer F.Cu) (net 14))
 (segment (start 167.64 104.14) (end 176.53 113.03) (width 0.25) (layer F.Cu) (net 14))
 (segment (start 167.64 103.873268) (end 167.64 104.14) (width 0.25) (layer F.Cu) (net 14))
 (segment (start 176.53 113.03) (end 177.8 113.03) (width 0.25) (layer F.Cu) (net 14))
 (segment (start 163.920322 100.79) (end 166.37 103.239678) (width 0.25) (layer F.Cu) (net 15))
 (segment (start 162.87 100.79) (end 163.920322 100.79) (width 0.25) (layer F.Cu) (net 15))
 (segment (start 166.37 105.41) (end 176.53 115.57) (width 0.25) (layer F.Cu) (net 15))
 (segment (start 166.37 103.239678) (end 166.37 105.41) (width 0.25) (layer F.Cu) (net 15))
 (segment (start 176.53 115.57) (end 177.8 115.57) (width 0.25) (layer F.Cu) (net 15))
 (segment (start 163.783912 101.29) (end 165.1 102.606088) (width 0.25) (layer F.Cu) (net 16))
 (segment (start 162.87 101.29) (end 163.783912 101.29) (width 0.25) (layer F.Cu) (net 16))
 (segment (start 165.1 106.68) (end 176.53 118.11) (width 0.25) (layer F.Cu) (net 16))
 (segment (start 165.1 102.606088) (end 165.1 106.68) (width 0.25) (layer F.Cu) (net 16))
 (segment (start 176.53 118.11) (end 177.8 118.11) (width 0.25) (layer F.Cu) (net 16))
 (segment (start 176.950001 119.800001) (end 177.8 120.65) (width 0.25) (layer F.Cu) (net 17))
 (segment (start 163.745001 107.865001) (end 175.680001 119.800001) (width 0.25) (layer F.Cu) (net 17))
 (segment (start 163.745001 101.887499) (end 163.745001 107.865001) (width 0.25) (layer F.Cu) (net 17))
 (segment (start 163.647502 101.79) (end 163.745001 101.887499) (width 0.25) (layer F.Cu) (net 17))
 (segment (start 162.87 101.79) (end 163.647502 101.79) (width 0.25) (layer F.Cu) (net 17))
 (segment (start 176.950001 119.800001) (end 175.680001 119.800001) (width 0.25) (layer F.Cu) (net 17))
 (segment (start 163.745001 92.794999) (end 175.680001 80.859999) (width 0.25) (layer F.Cu) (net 2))
 (segment (start 163.745001 93.692501) (end 163.745001 92.794999) (width 0.25) (layer F.Cu) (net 2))
 (segment (start 163.647502 93.79) (end 163.745001 93.692501) (width 0.25) (layer F.Cu) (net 2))
 (segment (start 176.950001 80.859999) (end 177.8 80.01) (width 0.25) (layer F.Cu) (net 2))
 (segment (start 162.87 93.79) (end 163.647502 93.79) (width 0.25) (layer F.Cu) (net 2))
 (segment (start 175.680001 80.859999) (end 176.950001 80.859999) (width 0.25) (layer F.Cu) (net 2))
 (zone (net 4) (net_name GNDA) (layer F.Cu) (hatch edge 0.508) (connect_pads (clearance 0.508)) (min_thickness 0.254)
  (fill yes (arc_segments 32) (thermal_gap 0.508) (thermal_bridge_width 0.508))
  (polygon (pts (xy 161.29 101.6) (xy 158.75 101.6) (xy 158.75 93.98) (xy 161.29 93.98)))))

